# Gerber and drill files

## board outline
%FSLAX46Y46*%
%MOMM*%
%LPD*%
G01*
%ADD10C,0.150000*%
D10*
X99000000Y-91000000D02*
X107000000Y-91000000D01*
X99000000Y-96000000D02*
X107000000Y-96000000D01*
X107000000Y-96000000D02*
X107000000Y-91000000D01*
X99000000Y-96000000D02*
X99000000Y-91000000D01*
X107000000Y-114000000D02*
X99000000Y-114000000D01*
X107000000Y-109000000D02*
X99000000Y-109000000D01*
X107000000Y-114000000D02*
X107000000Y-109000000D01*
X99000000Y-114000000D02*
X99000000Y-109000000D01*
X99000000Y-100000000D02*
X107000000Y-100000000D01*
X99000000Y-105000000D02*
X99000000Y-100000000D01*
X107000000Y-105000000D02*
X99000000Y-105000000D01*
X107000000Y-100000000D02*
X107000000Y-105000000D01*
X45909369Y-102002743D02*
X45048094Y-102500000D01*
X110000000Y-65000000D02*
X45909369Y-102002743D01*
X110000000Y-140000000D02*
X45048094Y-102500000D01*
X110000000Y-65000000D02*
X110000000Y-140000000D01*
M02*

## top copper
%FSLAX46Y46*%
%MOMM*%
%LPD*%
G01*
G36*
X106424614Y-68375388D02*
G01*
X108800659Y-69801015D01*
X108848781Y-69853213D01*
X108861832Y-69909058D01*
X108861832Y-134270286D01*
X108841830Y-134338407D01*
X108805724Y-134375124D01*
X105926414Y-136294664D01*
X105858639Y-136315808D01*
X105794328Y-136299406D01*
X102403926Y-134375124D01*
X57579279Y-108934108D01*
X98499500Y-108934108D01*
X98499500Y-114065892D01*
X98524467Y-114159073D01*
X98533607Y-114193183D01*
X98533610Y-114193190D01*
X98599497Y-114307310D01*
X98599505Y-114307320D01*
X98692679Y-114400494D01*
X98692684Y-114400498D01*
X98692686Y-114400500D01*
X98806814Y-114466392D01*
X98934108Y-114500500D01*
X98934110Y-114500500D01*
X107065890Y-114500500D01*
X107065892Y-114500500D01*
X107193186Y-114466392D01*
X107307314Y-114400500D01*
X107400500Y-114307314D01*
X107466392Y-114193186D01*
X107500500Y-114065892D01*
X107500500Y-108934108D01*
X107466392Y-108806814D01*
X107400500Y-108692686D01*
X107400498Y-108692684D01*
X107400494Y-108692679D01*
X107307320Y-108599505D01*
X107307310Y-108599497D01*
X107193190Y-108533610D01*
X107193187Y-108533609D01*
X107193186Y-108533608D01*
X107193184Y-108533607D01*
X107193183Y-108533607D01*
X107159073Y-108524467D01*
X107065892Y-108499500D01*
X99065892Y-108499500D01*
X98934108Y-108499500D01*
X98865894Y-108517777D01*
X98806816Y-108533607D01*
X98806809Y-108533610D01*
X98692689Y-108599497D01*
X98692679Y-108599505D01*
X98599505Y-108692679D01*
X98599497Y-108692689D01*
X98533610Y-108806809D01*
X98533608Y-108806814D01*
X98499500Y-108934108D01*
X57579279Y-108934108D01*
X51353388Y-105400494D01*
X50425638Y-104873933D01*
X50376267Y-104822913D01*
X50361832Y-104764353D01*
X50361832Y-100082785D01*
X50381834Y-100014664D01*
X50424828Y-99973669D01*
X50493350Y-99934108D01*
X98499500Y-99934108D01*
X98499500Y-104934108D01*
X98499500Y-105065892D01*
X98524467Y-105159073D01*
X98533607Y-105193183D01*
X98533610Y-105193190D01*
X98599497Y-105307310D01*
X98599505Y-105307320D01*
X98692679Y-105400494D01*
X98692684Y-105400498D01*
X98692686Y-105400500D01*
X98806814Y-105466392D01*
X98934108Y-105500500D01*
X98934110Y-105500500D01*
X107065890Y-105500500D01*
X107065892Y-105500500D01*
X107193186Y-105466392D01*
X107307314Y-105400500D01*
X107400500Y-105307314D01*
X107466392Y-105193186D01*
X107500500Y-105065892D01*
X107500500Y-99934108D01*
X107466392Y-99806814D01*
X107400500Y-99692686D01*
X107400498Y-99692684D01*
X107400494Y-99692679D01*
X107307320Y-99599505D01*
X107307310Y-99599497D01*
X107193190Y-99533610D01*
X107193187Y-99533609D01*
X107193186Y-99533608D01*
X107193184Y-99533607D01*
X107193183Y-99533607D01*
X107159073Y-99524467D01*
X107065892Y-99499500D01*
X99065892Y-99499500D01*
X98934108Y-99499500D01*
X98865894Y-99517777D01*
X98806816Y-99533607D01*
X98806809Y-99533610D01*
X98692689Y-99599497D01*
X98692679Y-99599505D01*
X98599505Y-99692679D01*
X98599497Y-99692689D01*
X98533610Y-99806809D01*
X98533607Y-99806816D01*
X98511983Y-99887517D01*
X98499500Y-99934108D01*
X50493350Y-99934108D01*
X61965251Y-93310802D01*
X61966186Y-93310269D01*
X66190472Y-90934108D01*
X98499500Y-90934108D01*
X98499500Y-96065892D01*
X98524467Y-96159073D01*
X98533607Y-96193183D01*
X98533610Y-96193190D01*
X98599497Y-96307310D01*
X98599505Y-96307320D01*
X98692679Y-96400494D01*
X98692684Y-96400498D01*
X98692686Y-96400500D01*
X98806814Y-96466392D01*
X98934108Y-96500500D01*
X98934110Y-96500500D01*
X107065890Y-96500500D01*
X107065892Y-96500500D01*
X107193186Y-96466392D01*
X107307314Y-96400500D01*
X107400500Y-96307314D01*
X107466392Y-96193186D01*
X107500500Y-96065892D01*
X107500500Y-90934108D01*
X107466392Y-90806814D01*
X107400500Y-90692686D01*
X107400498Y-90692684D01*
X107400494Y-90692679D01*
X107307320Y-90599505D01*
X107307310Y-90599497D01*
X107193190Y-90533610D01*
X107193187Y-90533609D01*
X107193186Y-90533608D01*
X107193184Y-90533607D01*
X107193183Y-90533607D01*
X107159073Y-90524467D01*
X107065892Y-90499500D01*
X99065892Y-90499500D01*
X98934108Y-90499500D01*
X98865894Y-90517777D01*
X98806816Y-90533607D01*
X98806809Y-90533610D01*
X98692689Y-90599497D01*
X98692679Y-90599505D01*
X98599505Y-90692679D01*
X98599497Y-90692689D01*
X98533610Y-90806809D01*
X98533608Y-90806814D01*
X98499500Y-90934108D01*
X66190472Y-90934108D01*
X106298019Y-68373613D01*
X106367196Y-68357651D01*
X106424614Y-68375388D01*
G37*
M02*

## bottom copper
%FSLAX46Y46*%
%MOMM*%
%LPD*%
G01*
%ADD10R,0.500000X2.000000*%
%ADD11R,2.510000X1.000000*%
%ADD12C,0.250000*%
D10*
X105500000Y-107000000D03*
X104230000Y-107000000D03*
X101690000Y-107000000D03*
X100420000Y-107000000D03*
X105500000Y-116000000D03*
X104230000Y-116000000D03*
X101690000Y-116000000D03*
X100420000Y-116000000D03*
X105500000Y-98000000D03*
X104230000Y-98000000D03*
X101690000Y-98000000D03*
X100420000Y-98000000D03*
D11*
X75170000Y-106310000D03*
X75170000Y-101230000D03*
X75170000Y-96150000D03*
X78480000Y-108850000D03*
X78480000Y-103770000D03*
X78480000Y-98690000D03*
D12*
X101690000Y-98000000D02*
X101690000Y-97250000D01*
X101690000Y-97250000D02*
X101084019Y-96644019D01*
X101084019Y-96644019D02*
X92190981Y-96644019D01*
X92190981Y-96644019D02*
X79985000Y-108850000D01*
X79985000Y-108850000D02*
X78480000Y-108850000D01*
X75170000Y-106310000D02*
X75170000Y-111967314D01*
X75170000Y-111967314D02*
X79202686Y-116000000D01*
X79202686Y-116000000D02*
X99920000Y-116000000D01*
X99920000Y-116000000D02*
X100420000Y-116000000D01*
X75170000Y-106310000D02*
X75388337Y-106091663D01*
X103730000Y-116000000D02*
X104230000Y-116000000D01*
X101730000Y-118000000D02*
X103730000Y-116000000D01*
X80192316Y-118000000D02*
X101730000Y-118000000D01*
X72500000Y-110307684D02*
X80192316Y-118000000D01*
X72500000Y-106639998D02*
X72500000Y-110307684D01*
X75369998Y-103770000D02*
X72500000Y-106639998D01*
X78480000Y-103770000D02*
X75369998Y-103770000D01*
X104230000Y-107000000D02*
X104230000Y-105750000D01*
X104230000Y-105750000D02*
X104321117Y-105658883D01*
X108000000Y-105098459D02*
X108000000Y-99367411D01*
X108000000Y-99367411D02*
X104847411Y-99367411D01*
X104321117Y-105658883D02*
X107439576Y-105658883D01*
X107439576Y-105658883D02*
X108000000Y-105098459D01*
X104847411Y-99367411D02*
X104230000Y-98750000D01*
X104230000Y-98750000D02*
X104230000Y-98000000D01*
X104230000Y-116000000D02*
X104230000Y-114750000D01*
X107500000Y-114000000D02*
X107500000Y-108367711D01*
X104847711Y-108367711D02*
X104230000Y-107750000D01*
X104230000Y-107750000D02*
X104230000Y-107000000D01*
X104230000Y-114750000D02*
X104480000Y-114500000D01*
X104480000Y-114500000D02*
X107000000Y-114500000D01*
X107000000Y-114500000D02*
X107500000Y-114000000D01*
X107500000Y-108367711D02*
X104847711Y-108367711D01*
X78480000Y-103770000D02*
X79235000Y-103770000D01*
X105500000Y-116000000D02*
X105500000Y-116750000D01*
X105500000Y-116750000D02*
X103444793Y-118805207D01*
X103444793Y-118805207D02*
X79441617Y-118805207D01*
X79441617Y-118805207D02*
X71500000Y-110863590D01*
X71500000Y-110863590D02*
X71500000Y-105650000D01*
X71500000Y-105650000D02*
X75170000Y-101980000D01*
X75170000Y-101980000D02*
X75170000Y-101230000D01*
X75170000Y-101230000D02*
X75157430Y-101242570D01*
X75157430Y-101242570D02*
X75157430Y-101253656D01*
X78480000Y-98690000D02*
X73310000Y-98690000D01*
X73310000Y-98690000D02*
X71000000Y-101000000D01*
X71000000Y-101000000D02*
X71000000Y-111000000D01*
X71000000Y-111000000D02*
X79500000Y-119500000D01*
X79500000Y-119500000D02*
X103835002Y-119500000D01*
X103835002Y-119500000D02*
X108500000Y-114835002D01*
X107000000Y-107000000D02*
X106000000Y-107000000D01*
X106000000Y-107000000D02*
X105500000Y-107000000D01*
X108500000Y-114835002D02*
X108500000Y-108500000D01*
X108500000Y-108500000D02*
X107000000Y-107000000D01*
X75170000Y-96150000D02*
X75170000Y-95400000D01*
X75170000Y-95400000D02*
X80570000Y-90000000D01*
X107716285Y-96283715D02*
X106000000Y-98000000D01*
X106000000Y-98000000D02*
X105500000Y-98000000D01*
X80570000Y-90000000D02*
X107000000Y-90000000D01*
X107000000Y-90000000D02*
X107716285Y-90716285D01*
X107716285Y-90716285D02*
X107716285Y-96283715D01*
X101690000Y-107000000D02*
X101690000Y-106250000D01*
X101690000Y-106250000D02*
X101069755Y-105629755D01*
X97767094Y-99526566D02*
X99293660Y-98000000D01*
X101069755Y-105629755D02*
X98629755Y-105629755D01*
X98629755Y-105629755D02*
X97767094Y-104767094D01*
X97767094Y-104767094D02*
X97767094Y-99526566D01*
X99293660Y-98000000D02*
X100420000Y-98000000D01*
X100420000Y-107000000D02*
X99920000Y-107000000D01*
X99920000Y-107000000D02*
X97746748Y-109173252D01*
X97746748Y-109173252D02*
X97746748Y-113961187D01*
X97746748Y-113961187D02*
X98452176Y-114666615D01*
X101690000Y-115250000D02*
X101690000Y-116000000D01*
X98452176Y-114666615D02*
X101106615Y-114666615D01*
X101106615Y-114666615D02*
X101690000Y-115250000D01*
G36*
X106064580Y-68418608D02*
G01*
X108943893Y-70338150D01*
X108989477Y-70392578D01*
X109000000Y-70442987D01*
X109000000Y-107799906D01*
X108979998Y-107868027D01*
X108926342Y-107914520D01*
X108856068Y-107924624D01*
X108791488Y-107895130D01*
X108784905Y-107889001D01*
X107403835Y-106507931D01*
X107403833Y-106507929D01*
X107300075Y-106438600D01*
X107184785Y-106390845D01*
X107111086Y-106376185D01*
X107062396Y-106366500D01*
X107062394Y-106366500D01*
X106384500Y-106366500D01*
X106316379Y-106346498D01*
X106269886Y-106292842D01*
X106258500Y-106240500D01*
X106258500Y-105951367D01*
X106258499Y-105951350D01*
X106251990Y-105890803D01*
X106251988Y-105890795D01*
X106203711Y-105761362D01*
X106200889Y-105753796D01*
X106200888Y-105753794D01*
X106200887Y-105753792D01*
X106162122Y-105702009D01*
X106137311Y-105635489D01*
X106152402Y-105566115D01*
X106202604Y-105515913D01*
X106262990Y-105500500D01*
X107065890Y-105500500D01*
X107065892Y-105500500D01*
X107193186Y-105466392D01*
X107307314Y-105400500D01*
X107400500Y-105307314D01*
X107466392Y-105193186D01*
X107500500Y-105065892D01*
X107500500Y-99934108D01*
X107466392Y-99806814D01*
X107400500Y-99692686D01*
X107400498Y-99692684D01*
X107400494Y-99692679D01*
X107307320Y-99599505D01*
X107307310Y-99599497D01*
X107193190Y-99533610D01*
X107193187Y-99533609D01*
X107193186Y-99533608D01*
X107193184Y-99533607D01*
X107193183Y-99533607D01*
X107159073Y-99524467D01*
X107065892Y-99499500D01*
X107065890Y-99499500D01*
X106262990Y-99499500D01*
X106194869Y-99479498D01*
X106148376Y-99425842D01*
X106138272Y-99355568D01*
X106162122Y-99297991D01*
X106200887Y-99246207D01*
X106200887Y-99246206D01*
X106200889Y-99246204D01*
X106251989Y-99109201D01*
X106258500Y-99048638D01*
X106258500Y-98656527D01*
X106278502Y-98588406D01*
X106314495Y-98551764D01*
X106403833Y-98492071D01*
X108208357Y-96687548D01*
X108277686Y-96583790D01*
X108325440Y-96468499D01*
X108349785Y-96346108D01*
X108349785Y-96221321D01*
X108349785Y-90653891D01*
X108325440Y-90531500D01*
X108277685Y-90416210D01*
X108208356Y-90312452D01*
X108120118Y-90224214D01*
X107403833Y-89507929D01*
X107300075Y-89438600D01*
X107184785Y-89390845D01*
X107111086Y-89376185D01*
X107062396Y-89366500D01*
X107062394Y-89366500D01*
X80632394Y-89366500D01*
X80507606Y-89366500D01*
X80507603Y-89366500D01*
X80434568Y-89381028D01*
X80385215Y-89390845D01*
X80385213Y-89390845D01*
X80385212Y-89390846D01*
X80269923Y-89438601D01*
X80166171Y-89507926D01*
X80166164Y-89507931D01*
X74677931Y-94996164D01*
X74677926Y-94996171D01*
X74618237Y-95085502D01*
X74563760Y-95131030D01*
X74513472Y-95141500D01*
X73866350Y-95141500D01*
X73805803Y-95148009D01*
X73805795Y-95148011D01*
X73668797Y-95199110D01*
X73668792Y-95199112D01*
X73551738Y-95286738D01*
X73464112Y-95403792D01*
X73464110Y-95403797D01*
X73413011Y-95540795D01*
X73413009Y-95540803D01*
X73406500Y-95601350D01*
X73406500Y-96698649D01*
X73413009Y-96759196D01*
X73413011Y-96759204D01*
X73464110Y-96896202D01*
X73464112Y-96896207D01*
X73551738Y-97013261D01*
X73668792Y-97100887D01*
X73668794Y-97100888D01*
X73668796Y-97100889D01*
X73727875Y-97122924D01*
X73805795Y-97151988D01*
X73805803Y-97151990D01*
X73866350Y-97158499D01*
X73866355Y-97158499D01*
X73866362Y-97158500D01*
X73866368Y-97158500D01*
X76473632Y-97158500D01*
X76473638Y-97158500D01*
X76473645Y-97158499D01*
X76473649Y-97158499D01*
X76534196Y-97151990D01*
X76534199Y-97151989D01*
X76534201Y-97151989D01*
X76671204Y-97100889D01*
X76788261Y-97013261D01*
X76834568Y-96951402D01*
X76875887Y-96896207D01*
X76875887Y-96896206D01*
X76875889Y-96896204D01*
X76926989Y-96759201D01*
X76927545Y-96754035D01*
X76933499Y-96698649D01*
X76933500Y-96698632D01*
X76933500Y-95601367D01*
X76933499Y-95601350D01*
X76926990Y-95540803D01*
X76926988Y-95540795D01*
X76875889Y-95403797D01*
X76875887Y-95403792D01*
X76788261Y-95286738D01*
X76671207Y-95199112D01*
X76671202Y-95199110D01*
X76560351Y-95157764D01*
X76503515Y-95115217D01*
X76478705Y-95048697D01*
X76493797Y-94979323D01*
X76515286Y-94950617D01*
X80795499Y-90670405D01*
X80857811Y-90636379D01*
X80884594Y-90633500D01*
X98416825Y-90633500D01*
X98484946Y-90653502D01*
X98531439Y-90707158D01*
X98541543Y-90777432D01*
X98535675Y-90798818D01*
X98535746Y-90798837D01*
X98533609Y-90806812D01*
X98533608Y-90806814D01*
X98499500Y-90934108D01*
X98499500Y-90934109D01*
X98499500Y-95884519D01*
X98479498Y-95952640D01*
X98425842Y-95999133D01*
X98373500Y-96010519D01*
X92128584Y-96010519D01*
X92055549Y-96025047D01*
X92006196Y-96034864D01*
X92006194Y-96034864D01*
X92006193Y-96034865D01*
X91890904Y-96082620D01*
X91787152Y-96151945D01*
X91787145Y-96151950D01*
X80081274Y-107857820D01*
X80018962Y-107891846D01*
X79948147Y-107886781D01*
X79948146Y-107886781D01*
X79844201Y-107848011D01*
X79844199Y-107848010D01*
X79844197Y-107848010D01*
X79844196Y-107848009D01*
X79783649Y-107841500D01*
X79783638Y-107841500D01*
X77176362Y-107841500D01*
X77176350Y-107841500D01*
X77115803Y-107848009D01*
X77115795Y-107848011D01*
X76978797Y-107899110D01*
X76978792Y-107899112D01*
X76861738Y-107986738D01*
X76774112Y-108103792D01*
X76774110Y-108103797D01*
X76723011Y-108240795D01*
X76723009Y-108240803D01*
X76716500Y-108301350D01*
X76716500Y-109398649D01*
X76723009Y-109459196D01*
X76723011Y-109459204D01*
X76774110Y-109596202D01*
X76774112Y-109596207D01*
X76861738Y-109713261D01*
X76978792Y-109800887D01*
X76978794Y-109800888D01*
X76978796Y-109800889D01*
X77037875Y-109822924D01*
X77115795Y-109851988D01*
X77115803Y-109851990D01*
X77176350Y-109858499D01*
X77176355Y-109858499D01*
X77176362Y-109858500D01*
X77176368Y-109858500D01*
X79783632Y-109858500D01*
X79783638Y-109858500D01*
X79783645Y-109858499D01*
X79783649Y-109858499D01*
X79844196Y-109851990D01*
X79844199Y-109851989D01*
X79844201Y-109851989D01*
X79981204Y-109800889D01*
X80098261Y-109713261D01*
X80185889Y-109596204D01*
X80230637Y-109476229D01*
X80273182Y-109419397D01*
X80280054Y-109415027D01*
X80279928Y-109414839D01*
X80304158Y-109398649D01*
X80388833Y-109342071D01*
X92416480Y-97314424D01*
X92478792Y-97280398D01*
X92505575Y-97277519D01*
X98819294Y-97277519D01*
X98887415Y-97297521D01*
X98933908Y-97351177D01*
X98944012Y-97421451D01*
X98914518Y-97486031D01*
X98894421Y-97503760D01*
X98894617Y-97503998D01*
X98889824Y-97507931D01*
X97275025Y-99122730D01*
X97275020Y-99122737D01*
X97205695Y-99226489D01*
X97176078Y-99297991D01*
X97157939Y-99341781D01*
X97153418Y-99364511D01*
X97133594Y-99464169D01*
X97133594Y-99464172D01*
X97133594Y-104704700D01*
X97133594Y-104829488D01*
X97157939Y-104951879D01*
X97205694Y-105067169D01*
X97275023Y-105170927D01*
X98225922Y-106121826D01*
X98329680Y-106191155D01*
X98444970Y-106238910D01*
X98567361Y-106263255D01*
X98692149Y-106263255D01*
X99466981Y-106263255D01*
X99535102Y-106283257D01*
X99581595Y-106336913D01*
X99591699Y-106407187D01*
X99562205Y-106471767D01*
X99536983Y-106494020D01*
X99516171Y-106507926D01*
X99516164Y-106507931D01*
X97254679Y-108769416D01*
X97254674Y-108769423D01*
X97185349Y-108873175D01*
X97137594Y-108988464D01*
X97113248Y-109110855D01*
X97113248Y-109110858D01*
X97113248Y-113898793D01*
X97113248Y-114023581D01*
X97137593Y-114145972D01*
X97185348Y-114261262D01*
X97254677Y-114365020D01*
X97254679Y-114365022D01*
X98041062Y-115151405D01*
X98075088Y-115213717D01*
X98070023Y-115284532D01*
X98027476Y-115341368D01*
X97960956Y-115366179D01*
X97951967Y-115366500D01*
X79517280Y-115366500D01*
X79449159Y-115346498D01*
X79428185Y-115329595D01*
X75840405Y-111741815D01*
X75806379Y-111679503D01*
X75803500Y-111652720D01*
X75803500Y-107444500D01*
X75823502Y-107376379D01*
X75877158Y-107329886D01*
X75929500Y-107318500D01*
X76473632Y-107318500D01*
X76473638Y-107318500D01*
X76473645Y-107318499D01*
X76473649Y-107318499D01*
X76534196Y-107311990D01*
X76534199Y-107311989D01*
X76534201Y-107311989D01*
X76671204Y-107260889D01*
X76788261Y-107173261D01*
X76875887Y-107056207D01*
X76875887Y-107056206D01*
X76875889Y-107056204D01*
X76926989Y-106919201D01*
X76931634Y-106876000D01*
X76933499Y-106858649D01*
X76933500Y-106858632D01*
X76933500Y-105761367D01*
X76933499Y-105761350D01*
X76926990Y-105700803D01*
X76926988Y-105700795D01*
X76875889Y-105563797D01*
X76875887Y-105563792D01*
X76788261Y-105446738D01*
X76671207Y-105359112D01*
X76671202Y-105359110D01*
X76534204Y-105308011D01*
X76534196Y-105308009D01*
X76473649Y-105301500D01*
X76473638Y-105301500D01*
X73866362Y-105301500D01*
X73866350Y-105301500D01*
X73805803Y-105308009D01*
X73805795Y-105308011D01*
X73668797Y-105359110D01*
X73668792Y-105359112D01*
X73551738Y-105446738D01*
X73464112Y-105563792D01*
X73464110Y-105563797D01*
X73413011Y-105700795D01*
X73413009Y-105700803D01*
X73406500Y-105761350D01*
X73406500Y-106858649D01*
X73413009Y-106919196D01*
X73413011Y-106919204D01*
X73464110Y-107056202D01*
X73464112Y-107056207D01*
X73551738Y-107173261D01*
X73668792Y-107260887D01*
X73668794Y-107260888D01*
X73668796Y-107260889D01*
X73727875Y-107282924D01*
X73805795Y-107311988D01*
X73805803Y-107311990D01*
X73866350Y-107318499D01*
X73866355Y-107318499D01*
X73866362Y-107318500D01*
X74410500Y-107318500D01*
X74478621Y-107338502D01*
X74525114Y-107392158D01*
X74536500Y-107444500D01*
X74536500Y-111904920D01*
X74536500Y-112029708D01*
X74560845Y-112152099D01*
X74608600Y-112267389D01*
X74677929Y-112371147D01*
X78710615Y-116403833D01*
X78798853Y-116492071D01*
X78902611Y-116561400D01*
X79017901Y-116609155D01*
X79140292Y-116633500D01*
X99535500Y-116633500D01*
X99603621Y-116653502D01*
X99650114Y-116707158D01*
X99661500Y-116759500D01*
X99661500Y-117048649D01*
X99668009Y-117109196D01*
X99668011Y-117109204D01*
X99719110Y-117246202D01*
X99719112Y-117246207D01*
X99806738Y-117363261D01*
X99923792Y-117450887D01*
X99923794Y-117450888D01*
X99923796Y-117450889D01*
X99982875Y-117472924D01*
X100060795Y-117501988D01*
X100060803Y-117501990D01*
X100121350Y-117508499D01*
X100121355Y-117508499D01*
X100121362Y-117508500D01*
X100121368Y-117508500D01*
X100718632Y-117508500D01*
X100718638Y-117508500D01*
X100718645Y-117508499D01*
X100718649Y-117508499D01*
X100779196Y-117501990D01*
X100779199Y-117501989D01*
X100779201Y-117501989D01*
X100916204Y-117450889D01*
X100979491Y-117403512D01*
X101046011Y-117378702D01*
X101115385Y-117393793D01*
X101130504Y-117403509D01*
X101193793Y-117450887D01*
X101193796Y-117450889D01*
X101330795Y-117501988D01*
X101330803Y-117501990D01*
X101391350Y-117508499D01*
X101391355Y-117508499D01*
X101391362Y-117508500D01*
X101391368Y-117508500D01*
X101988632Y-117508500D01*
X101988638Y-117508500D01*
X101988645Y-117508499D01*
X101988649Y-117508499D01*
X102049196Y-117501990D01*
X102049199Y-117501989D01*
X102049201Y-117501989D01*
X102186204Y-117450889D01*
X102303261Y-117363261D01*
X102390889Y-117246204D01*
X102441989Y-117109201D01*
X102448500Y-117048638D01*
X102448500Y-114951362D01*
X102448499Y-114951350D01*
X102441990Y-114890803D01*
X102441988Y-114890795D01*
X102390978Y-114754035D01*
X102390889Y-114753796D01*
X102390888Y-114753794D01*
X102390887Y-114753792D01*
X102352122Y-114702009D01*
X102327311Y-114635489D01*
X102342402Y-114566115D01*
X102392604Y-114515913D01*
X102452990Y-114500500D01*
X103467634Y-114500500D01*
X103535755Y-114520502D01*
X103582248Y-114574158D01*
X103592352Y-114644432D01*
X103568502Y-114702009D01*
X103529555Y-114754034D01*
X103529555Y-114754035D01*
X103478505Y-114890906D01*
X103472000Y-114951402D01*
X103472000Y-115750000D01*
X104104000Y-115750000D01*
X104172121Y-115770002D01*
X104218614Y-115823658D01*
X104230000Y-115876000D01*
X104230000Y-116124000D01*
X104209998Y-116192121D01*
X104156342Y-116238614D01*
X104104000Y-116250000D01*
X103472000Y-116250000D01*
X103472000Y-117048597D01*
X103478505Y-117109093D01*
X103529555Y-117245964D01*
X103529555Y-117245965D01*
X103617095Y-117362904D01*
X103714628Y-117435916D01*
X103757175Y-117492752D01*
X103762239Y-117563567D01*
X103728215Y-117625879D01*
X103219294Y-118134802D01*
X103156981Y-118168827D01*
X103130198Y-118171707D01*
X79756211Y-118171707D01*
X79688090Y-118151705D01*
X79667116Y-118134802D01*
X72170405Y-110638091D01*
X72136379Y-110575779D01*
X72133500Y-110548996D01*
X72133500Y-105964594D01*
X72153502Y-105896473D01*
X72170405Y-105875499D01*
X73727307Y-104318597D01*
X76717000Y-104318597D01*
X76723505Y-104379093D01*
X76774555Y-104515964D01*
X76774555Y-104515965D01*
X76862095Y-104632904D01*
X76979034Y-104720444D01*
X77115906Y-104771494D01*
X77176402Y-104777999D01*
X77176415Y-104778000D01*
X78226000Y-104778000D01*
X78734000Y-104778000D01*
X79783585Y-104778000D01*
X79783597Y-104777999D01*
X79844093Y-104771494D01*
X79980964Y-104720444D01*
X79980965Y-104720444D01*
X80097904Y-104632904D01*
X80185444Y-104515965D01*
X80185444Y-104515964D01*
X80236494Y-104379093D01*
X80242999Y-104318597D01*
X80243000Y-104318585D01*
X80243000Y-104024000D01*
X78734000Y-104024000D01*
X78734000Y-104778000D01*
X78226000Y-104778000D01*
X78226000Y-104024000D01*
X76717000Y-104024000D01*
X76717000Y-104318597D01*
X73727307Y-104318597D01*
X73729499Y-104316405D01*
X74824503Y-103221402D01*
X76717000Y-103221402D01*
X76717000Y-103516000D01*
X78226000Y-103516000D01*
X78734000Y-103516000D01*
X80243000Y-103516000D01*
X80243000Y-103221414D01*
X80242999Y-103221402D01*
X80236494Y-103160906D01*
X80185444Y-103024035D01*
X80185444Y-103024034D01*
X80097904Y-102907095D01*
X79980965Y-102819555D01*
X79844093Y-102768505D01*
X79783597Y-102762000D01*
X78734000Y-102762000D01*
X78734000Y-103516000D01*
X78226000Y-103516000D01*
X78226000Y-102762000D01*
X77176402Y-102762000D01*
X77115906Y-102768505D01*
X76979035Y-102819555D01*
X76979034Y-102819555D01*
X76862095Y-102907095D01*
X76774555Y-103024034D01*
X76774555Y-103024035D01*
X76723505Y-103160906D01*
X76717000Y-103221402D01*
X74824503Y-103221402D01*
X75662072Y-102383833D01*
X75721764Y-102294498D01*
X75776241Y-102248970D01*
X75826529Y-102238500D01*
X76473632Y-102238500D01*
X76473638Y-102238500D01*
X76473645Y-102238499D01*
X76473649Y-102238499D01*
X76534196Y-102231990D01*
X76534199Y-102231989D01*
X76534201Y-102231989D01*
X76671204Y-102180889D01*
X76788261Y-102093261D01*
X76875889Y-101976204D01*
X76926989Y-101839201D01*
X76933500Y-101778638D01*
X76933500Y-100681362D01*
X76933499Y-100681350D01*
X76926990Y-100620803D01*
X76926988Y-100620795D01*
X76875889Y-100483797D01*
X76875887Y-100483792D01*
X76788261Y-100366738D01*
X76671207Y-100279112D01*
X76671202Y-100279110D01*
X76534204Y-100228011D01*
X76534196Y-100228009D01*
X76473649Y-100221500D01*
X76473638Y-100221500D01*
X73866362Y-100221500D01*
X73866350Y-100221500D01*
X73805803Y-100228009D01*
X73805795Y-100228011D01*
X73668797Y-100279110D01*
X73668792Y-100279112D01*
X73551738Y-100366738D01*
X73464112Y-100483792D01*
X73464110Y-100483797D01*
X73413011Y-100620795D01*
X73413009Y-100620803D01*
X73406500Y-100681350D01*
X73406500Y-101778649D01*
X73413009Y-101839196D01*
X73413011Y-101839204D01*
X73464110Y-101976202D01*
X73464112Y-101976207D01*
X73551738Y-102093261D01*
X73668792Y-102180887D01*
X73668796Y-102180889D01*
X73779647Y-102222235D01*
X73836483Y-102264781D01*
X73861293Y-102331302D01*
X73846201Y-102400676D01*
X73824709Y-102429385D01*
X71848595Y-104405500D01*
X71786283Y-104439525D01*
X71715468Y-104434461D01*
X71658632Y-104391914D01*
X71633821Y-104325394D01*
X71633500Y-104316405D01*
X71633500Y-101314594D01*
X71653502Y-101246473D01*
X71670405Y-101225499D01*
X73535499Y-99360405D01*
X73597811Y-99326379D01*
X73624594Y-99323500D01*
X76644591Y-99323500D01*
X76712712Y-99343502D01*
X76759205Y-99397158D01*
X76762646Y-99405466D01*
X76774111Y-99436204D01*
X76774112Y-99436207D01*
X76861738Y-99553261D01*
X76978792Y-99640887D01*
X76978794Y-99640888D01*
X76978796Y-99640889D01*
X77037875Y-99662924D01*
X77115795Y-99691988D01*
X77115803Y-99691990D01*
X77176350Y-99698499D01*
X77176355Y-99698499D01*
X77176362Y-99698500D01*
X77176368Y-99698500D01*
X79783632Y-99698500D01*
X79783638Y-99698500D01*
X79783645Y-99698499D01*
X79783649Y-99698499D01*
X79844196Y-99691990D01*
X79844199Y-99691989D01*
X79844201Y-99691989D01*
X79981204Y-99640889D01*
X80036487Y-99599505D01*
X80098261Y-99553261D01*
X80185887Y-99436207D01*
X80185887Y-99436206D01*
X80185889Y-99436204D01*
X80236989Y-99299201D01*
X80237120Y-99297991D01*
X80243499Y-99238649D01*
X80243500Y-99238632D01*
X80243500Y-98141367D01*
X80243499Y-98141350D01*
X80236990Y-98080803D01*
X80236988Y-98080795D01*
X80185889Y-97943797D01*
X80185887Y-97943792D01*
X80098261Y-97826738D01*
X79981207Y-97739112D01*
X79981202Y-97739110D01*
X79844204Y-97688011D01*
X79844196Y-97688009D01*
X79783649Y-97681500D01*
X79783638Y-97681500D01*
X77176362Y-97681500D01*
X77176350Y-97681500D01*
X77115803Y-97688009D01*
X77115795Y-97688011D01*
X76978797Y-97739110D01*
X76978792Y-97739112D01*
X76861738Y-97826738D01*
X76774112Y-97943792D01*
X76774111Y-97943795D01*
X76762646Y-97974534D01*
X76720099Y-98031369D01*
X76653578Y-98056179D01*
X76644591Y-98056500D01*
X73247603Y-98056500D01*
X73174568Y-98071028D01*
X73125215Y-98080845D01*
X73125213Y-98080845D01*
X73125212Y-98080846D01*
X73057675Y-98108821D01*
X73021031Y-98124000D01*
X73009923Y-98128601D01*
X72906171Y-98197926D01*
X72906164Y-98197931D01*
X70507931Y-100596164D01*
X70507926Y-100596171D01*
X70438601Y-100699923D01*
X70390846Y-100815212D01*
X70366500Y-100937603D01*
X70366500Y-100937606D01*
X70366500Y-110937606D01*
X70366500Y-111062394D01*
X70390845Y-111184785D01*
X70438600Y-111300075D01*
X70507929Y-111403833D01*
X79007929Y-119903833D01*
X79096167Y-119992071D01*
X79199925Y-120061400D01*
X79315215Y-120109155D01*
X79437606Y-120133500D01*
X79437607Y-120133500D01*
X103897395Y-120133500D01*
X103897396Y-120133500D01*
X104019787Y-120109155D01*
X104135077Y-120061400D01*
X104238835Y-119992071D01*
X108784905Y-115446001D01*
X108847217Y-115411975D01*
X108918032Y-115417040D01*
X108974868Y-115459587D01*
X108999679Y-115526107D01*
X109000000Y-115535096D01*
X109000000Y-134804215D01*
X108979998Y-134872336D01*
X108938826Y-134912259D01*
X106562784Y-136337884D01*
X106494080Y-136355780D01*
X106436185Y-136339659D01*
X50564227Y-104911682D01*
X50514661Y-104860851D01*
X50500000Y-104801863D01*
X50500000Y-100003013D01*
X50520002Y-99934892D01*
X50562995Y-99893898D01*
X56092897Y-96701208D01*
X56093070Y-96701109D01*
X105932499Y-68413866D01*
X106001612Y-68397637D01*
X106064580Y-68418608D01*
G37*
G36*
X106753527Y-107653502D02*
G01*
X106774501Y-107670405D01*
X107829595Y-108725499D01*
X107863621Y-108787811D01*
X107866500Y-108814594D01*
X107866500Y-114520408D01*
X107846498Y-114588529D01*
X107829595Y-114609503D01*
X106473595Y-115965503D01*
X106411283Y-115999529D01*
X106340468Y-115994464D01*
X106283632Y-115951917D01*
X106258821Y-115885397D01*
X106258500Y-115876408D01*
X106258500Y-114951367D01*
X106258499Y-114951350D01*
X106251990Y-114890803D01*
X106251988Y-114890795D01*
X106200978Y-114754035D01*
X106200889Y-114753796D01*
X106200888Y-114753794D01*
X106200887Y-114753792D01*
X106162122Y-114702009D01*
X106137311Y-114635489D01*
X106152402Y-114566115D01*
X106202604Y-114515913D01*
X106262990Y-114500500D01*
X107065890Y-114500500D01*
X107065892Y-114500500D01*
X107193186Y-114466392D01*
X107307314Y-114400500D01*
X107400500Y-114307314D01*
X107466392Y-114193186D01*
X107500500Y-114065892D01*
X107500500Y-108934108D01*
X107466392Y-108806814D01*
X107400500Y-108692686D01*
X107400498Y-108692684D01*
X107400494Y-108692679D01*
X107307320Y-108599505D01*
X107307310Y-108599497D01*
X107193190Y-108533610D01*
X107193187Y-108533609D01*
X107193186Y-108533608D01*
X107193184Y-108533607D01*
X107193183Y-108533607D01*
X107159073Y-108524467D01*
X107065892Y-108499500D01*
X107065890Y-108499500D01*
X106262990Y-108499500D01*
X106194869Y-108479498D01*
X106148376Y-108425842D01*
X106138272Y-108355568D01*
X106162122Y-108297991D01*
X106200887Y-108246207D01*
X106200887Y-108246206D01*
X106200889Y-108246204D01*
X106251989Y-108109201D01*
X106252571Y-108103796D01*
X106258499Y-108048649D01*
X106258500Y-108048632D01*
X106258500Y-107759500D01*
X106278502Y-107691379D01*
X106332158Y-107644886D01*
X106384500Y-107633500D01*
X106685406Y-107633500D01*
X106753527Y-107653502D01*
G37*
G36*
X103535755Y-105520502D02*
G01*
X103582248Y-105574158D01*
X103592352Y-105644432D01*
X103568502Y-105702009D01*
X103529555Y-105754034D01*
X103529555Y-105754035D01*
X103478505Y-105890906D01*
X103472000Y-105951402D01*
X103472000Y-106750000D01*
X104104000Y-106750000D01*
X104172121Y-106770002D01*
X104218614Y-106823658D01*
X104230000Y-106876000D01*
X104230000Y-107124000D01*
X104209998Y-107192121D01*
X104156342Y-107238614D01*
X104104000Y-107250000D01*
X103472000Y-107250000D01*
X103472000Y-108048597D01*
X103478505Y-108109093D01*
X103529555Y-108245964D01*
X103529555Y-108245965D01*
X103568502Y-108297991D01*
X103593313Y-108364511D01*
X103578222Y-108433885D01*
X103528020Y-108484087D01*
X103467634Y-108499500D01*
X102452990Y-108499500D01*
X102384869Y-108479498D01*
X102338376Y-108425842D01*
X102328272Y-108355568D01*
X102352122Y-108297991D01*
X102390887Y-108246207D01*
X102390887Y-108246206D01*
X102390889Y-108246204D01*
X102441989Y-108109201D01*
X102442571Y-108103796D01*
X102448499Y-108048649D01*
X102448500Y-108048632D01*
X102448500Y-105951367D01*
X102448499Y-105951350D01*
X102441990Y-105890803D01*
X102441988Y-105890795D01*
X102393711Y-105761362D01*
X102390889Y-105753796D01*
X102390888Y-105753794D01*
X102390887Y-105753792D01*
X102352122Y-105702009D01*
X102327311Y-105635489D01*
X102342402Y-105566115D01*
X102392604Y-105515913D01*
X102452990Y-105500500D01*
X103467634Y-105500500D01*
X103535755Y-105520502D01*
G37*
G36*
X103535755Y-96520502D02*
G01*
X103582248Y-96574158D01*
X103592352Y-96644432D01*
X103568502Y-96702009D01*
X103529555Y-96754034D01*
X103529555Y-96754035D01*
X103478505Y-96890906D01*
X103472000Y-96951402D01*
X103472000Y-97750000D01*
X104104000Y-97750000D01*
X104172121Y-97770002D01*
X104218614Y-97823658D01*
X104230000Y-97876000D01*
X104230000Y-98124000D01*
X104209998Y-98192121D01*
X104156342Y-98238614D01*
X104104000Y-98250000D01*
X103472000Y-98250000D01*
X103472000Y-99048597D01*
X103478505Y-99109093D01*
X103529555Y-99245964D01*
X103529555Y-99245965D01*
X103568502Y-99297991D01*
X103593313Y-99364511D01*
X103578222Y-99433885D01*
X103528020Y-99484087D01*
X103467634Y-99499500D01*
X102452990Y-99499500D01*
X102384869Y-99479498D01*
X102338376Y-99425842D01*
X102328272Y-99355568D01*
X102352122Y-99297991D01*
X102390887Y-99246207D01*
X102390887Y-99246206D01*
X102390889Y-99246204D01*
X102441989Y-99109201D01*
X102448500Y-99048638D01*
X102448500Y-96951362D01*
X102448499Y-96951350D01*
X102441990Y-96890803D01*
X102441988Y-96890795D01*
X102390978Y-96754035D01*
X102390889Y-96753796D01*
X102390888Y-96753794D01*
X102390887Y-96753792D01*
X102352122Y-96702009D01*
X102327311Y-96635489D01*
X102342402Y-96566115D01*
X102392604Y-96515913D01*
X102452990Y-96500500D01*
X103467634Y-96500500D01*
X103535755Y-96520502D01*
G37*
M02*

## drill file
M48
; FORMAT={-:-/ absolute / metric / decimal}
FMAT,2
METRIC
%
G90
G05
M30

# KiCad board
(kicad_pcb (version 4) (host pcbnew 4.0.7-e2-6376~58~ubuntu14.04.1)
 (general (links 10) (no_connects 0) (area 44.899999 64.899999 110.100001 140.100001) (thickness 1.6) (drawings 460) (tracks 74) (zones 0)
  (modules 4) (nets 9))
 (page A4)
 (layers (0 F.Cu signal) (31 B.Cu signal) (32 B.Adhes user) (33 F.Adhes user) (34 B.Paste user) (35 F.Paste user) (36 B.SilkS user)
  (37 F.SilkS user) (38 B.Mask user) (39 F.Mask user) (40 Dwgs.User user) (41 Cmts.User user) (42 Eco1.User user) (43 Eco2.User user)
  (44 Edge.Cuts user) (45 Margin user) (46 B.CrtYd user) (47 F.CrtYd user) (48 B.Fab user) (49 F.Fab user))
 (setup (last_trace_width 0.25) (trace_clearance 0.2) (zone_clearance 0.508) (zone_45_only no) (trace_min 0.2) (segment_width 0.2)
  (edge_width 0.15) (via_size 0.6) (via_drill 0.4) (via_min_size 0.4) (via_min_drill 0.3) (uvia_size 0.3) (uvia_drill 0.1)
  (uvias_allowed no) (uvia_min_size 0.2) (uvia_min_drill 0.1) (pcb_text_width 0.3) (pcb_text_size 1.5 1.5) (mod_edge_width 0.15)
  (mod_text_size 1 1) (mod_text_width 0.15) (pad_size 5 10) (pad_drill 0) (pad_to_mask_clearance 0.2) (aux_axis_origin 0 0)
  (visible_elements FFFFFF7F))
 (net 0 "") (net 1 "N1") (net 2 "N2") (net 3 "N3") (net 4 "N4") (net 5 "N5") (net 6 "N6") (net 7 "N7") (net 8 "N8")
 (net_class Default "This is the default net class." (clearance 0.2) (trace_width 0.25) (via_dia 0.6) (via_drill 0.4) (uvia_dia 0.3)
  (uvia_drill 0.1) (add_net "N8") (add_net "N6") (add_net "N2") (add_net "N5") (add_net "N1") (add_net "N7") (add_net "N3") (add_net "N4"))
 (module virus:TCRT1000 (layer B.Cu) (at 103.5 109 180)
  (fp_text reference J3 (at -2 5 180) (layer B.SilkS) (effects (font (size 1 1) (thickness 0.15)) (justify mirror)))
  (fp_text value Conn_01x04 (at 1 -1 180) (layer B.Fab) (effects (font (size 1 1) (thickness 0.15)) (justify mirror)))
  (pad 1 smd rect (at -2 2 180) (size 0.5 2) (layers B.Cu B.Paste B.Mask) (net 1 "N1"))
  (pad 2 smd rect (at -0.73 2 180) (size 0.5 2) (layers B.Cu B.Paste B.Mask) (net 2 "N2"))
  (pad 3 smd rect (at 1.81 2 180) (size 0.5 2) (layers B.Cu B.Paste B.Mask) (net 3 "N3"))
  (pad 4 smd rect (at 3.08 2 180) (size 0.5 2) (layers B.Cu B.Paste B.Mask) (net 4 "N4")))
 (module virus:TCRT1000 (layer B.Cu) (at 103.5 118 180)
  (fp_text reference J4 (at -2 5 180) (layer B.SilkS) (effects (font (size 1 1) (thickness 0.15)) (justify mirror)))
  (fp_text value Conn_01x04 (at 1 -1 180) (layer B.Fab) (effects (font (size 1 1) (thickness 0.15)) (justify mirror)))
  (pad 1 smd rect (at -2 2 180) (size 0.5 2) (layers B.Cu B.Paste B.Mask) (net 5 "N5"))
  (pad 2 smd rect (at -0.73 2 180) (size 0.5 2) (layers B.Cu B.Paste B.Mask) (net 2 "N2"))
  (pad 3 smd rect (at 1.81 2 180) (size 0.5 2) (layers B.Cu B.Paste B.Mask) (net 4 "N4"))
  (pad 4 smd rect (at 3.08 2 180) (size 0.5 2) (layers B.Cu B.Paste B.Mask) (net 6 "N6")))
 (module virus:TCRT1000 (layer B.Cu) (at 103.5 100 180)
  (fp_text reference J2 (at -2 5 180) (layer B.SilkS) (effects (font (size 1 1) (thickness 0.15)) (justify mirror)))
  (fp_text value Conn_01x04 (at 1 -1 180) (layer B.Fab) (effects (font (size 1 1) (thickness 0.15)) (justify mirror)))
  (pad 1 smd rect (at -2 2 180) (size 0.5 2) (layers B.Cu B.Paste B.Mask) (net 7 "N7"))
  (pad 2 smd rect (at -0.73 2 180) (size 0.5 2) (layers B.Cu B.Paste B.Mask) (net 2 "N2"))
  (pad 3 smd rect (at 1.81 2 180) (size 0.5 2) (layers B.Cu B.Paste B.Mask) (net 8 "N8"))
  (pad 4 smd rect (at 3.08 2 180) (size 0.5 2) (layers B.Cu B.Paste B.Mask) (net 3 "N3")))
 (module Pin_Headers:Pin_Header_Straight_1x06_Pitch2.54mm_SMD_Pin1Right (layer B.Cu) (at 76.825 102.5)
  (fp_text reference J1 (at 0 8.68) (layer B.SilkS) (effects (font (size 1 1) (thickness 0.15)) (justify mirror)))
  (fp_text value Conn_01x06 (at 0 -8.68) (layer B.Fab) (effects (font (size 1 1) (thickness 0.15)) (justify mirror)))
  (pad 2 smd rect (at -1.655 3.81) (size 2.51 1) (layers B.Cu B.Paste B.Mask) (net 6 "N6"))
  (pad 4 smd rect (at -1.655 -1.27) (size 2.51 1) (layers B.Cu B.Paste B.Mask) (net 5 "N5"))
  (pad 6 smd rect (at -1.655 -6.35) (size 2.51 1) (layers B.Cu B.Paste B.Mask) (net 7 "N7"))
  (pad 1 smd rect (at 1.655 6.35) (size 2.51 1) (layers B.Cu B.Paste B.Mask) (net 8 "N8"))
  (pad 3 smd rect (at 1.655 1.27) (size 2.51 1) (layers B.Cu B.Paste B.Mask) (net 2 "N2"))
  (pad 5 smd rect (at 1.655 -3.81) (size 2.51 1) (layers B.Cu B.Paste B.Mask) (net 1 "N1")))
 (gr_line (start 99 91) (end 107 91) (layer Edge.Cuts) (width 0.15))
 (gr_line (start 99 96) (end 107 96) (layer Edge.Cuts) (width 0.15))
 (gr_line (start 107 96) (end 107 91) (layer Edge.Cuts) (width 0.15))
 (gr_line (start 99 96) (end 99 91) (layer Edge.Cuts) (width 0.15))
 (gr_line (start 107 114) (end 99 114) (layer Edge.Cuts) (width 0.15))
 (gr_line (start 107 109) (end 99 109) (layer Edge.Cuts) (width 0.15))
 (gr_line (start 107 114) (end 107 109) (layer Edge.Cuts) (width 0.15))
 (gr_line (start 99 114) (end 99 109) (layer Edge.Cuts) (width 0.15))
 (gr_line (start 99 100) (end 107 100) (layer Edge.Cuts) (width 0.15))
 (gr_line (start 99 105) (end 99 100) (layer Edge.Cuts) (width 0.15))
 (gr_line (start 107 105) (end 99 105) (layer Edge.Cuts) (width 0.15))
 (gr_line (start 107 100) (end 107 105) (layer Edge.Cuts) (width 0.15))
 (gr_line (start 45.909369 102.002743) (end 45.048094 102.5) (layer Edge.Cuts) (width 0.15))
 (gr_line (start 110 65) (end 45.909369 102.002743) (layer Edge.Cuts) (width 0.15))
 (gr_line (start 110 140) (end 45.048094 102.5) (layer Edge.Cuts) (width 0.15))
 (gr_line (start 110 65) (end 110 140) (layer Edge.Cuts) (width 0.15))
 (segment (start 101.69 98) (end 101.69 97.25) (width 0.25) (layer B.Cu) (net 8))
 (segment (start 101.69 97.25) (end 101.084019 96.644019) (width 0.25) (layer B.Cu) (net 8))
 (segment (start 101.084019 96.644019) (end 92.190981 96.644019) (width 0.25) (layer B.Cu) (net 8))
 (segment (start 92.190981 96.644019) (end 79.985 108.85) (width 0.25) (layer B.Cu) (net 8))
 (segment (start 79.985 108.85) (end 78.48 108.85) (width 0.25) (layer B.Cu) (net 8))
 (segment (start 75.17 106.31) (end 75.17 111.967314) (width 0.25) (layer B.Cu) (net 6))
 (segment (start 75.17 111.967314) (end 79.202686 116) (width 0.25) (layer B.Cu) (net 6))
 (segment (start 79.202686 116) (end 99.92 116) (width 0.25) (layer B.Cu) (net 6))
 (segment (start 99.92 116) (end 100.42 116) (width 0.25) (layer B.Cu) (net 6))
 (segment (start 75.17 106.31) (end 75.388337 106.091663) (width 0.25) (layer B.Cu) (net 6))
 (segment (start 103.73 116) (end 104.23 116) (width 0.25) (layer B.Cu) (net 2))
 (segment (start 101.73 118) (end 103.73 116) (width 0.25) (layer B.Cu) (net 2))
 (segment (start 80.192316 118) (end 101.73 118) (width 0.25) (layer B.Cu) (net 2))
 (segment (start 72.5 110.307684) (end 80.192316 118) (width 0.25) (layer B.Cu) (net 2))
 (segment (start 72.5 106.639998) (end 72.5 110.307684) (width 0.25) (layer B.Cu) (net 2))
 (segment (start 75.369998 103.77) (end 72.5 106.639998) (width 0.25) (layer B.Cu) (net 2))
 (segment (start 78.48 103.77) (end 75.369998 103.77) (width 0.25) (layer B.Cu) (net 2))
 (segment (start 104.23 107) (end 104.23 105.75) (width 0.25) (layer B.Cu) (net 2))
 (segment (start 104.23 105.75) (end 104.321117 105.658883) (width 0.25) (layer B.Cu) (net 2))
 (segment (start 108 105.098459) (end 108 99.367411) (width 0.25) (layer B.Cu) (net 2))
 (segment (start 108 99.367411) (end 104.847411 99.367411) (width 0.25) (layer B.Cu) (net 2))
 (segment (start 104.321117 105.658883) (end 107.439576 105.658883) (width 0.25) (layer B.Cu) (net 2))
 (segment (start 107.439576 105.658883) (end 108 105.098459) (width 0.25) (layer B.Cu) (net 2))
 (segment (start 104.847411 99.367411) (end 104.23 98.75) (width 0.25) (layer B.Cu) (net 2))
 (segment (start 104.23 98.75) (end 104.23 98) (width 0.25) (layer B.Cu) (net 2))
 (segment (start 104.23 116) (end 104.23 114.75) (width 0.25) (layer B.Cu) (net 2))
 (segment (start 107.5 114) (end 107.5 108.367711) (width 0.25) (layer B.Cu) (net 2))
 (segment (start 104.847711 108.367711) (end 104.23 107.75) (width 0.25) (layer B.Cu) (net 2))
 (segment (start 104.23 107.75) (end 104.23 107) (width 0.25) (layer B.Cu) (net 2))
 (segment (start 104.23 114.75) (end 104.48 114.5) (width 0.25) (layer B.Cu) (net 2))
 (segment (start 104.48 114.5) (end 107 114.5) (width 0.25) (layer B.Cu) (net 2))
 (segment (start 107 114.5) (end 107.5 114) (width 0.25) (layer B.Cu) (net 2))
 (segment (start 107.5 108.367711) (end 104.847711 108.367711) (width 0.25) (layer B.Cu) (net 2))
 (segment (start 78.48 103.77) (end 79.235 103.77) (width 0.25) (layer B.Cu) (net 2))
 (segment (start 105.5 116) (end 105.5 116.75) (width 0.25) (layer B.Cu) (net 5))
 (segment (start 105.5 116.75) (end 103.444793 118.805207) (width 0.25) (layer B.Cu) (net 5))
 (segment (start 103.444793 118.805207) (end 79.441617 118.805207) (width 0.25) (layer B.Cu) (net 5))
 (segment (start 79.441617 118.805207) (end 71.5 110.86359) (width 0.25) (layer B.Cu) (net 5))
 (segment (start 71.5 110.86359) (end 71.5 105.65) (width 0.25) (layer B.Cu) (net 5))
 (segment (start 71.5 105.65) (end 75.17 101.98) (width 0.25) (layer B.Cu) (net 5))
 (segment (start 75.17 101.98) (end 75.17 101.23) (width 0.25) (layer B.Cu) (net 5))
 (segment (start 75.17 101.23) (end 75.15743 101.24257) (width 0.25) (layer B.Cu) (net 5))
 (segment (start 75.15743 101.24257) (end 75.15743 101.253656) (width 0.25) (layer B.Cu) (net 5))
 (segment (start 78.48 98.69) (end 73.31 98.69) (width 0.25) (layer B.Cu) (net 1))
 (segment (start 73.31 98.69) (end 71 101) (width 0.25) (layer B.Cu) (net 1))
 (segment (start 71 101) (end 71 111) (width 0.25) (layer B.Cu) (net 1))
 (segment (start 71 111) (end 79.5 119.5) (width 0.25) (layer B.Cu) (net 1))
 (segment (start 79.5 119.5) (end 103.835002 119.5) (width 0.25) (layer B.Cu) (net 1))
 (segment (start 103.835002 119.5) (end 108.5 114.835002) (width 0.25) (layer B.Cu) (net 1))
 (segment (start 107 107) (end 106 107) (width 0.25) (layer B.Cu) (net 1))
 (segment (start 106 107) (end 105.5 107) (width 0.25) (layer B.Cu) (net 1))
 (segment (start 108.5 114.835002) (end 108.5 108.5) (width 0.25) (layer B.Cu) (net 1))
 (segment (start 108.5 108.5) (end 107 107) (width 0.25) (layer B.Cu) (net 1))
 (segment (start 75.17 96.15) (end 75.17 95.4) (width 0.25) (layer B.Cu) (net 7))
 (segment (start 75.17 95.4) (end 80.57 90) (width 0.25) (layer B.Cu) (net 7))
 (segment (start 107.716285 96.283715) (end 106 98) (width 0.25) (layer B.Cu) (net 7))
 (segment (start 106 98) (end 105.5 98) (width 0.25) (layer B.Cu) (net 7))
 (segment (start 80.57 90) (end 107 90) (width 0.25) (layer B.Cu) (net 7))
 (segment (start 107 90) (end 107.716285 90.716285) (width 0.25) (layer B.Cu) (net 7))
 (segment (start 107.716285 90.716285) (end 107.716285 96.283715) (width 0.25) (layer B.Cu) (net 7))
 (segment (start 101.69 107) (end 101.69 106.25) (width 0.25) (layer B.Cu) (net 3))
 (segment (start 101.69 106.25) (end 101.069755 105.629755) (width 0.25) (layer B.Cu) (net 3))
 (segment (start 97.767094 99.526566) (end 99.29366 98) (width 0.25) (layer B.Cu) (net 3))
 (segment (start 101.069755 105.629755) (end 98.629755 105.629755) (width 0.25) (layer B.Cu) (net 3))
 (segment (start 98.629755 105.629755) (end 97.767094 104.767094) (width 0.25) (layer B.Cu) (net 3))
 (segment (start 97.767094 104.767094) (end 97.767094 99.526566) (width 0.25) (layer B.Cu) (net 3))
 (segment (start 99.29366 98) (end 100.42 98) (width 0.25) (layer B.Cu) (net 3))
 (segment (start 100.42 107) (end 99.92 107) (width 0.25) (layer B.Cu) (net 4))
 (segment (start 99.92 107) (end 97.746748 109.173252) (width 0.25) (layer B.Cu) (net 4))
 (segment (start 97.746748 109.173252) (end 97.746748 113.961187) (width 0.25) (layer B.Cu) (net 4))
 (segment (start 97.746748 113.961187) (end 98.452176 114.666615) (width 0.25) (layer B.Cu) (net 4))
 (segment (start 101.69 115.25) (end 101.69 116) (width 0.25) (layer B.Cu) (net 4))
 (segment (start 98.452176 114.666615) (end 101.106615 114.666615) (width 0.25) (layer B.Cu) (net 4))
 (segment (start 101.106615 114.666615) (end 101.69 115.25) (width 0.25) (layer B.Cu) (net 4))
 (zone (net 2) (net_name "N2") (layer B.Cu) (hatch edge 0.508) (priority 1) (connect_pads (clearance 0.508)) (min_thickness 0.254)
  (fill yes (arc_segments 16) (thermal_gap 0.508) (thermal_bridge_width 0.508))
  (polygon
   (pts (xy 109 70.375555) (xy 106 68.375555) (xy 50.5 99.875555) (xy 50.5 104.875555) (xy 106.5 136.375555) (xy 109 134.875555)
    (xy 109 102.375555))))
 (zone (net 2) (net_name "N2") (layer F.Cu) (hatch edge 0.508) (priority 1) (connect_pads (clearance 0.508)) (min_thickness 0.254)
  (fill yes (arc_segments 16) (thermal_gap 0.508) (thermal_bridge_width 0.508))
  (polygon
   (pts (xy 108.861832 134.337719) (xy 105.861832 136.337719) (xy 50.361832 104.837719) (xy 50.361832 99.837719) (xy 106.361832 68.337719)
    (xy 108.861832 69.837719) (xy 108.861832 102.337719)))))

